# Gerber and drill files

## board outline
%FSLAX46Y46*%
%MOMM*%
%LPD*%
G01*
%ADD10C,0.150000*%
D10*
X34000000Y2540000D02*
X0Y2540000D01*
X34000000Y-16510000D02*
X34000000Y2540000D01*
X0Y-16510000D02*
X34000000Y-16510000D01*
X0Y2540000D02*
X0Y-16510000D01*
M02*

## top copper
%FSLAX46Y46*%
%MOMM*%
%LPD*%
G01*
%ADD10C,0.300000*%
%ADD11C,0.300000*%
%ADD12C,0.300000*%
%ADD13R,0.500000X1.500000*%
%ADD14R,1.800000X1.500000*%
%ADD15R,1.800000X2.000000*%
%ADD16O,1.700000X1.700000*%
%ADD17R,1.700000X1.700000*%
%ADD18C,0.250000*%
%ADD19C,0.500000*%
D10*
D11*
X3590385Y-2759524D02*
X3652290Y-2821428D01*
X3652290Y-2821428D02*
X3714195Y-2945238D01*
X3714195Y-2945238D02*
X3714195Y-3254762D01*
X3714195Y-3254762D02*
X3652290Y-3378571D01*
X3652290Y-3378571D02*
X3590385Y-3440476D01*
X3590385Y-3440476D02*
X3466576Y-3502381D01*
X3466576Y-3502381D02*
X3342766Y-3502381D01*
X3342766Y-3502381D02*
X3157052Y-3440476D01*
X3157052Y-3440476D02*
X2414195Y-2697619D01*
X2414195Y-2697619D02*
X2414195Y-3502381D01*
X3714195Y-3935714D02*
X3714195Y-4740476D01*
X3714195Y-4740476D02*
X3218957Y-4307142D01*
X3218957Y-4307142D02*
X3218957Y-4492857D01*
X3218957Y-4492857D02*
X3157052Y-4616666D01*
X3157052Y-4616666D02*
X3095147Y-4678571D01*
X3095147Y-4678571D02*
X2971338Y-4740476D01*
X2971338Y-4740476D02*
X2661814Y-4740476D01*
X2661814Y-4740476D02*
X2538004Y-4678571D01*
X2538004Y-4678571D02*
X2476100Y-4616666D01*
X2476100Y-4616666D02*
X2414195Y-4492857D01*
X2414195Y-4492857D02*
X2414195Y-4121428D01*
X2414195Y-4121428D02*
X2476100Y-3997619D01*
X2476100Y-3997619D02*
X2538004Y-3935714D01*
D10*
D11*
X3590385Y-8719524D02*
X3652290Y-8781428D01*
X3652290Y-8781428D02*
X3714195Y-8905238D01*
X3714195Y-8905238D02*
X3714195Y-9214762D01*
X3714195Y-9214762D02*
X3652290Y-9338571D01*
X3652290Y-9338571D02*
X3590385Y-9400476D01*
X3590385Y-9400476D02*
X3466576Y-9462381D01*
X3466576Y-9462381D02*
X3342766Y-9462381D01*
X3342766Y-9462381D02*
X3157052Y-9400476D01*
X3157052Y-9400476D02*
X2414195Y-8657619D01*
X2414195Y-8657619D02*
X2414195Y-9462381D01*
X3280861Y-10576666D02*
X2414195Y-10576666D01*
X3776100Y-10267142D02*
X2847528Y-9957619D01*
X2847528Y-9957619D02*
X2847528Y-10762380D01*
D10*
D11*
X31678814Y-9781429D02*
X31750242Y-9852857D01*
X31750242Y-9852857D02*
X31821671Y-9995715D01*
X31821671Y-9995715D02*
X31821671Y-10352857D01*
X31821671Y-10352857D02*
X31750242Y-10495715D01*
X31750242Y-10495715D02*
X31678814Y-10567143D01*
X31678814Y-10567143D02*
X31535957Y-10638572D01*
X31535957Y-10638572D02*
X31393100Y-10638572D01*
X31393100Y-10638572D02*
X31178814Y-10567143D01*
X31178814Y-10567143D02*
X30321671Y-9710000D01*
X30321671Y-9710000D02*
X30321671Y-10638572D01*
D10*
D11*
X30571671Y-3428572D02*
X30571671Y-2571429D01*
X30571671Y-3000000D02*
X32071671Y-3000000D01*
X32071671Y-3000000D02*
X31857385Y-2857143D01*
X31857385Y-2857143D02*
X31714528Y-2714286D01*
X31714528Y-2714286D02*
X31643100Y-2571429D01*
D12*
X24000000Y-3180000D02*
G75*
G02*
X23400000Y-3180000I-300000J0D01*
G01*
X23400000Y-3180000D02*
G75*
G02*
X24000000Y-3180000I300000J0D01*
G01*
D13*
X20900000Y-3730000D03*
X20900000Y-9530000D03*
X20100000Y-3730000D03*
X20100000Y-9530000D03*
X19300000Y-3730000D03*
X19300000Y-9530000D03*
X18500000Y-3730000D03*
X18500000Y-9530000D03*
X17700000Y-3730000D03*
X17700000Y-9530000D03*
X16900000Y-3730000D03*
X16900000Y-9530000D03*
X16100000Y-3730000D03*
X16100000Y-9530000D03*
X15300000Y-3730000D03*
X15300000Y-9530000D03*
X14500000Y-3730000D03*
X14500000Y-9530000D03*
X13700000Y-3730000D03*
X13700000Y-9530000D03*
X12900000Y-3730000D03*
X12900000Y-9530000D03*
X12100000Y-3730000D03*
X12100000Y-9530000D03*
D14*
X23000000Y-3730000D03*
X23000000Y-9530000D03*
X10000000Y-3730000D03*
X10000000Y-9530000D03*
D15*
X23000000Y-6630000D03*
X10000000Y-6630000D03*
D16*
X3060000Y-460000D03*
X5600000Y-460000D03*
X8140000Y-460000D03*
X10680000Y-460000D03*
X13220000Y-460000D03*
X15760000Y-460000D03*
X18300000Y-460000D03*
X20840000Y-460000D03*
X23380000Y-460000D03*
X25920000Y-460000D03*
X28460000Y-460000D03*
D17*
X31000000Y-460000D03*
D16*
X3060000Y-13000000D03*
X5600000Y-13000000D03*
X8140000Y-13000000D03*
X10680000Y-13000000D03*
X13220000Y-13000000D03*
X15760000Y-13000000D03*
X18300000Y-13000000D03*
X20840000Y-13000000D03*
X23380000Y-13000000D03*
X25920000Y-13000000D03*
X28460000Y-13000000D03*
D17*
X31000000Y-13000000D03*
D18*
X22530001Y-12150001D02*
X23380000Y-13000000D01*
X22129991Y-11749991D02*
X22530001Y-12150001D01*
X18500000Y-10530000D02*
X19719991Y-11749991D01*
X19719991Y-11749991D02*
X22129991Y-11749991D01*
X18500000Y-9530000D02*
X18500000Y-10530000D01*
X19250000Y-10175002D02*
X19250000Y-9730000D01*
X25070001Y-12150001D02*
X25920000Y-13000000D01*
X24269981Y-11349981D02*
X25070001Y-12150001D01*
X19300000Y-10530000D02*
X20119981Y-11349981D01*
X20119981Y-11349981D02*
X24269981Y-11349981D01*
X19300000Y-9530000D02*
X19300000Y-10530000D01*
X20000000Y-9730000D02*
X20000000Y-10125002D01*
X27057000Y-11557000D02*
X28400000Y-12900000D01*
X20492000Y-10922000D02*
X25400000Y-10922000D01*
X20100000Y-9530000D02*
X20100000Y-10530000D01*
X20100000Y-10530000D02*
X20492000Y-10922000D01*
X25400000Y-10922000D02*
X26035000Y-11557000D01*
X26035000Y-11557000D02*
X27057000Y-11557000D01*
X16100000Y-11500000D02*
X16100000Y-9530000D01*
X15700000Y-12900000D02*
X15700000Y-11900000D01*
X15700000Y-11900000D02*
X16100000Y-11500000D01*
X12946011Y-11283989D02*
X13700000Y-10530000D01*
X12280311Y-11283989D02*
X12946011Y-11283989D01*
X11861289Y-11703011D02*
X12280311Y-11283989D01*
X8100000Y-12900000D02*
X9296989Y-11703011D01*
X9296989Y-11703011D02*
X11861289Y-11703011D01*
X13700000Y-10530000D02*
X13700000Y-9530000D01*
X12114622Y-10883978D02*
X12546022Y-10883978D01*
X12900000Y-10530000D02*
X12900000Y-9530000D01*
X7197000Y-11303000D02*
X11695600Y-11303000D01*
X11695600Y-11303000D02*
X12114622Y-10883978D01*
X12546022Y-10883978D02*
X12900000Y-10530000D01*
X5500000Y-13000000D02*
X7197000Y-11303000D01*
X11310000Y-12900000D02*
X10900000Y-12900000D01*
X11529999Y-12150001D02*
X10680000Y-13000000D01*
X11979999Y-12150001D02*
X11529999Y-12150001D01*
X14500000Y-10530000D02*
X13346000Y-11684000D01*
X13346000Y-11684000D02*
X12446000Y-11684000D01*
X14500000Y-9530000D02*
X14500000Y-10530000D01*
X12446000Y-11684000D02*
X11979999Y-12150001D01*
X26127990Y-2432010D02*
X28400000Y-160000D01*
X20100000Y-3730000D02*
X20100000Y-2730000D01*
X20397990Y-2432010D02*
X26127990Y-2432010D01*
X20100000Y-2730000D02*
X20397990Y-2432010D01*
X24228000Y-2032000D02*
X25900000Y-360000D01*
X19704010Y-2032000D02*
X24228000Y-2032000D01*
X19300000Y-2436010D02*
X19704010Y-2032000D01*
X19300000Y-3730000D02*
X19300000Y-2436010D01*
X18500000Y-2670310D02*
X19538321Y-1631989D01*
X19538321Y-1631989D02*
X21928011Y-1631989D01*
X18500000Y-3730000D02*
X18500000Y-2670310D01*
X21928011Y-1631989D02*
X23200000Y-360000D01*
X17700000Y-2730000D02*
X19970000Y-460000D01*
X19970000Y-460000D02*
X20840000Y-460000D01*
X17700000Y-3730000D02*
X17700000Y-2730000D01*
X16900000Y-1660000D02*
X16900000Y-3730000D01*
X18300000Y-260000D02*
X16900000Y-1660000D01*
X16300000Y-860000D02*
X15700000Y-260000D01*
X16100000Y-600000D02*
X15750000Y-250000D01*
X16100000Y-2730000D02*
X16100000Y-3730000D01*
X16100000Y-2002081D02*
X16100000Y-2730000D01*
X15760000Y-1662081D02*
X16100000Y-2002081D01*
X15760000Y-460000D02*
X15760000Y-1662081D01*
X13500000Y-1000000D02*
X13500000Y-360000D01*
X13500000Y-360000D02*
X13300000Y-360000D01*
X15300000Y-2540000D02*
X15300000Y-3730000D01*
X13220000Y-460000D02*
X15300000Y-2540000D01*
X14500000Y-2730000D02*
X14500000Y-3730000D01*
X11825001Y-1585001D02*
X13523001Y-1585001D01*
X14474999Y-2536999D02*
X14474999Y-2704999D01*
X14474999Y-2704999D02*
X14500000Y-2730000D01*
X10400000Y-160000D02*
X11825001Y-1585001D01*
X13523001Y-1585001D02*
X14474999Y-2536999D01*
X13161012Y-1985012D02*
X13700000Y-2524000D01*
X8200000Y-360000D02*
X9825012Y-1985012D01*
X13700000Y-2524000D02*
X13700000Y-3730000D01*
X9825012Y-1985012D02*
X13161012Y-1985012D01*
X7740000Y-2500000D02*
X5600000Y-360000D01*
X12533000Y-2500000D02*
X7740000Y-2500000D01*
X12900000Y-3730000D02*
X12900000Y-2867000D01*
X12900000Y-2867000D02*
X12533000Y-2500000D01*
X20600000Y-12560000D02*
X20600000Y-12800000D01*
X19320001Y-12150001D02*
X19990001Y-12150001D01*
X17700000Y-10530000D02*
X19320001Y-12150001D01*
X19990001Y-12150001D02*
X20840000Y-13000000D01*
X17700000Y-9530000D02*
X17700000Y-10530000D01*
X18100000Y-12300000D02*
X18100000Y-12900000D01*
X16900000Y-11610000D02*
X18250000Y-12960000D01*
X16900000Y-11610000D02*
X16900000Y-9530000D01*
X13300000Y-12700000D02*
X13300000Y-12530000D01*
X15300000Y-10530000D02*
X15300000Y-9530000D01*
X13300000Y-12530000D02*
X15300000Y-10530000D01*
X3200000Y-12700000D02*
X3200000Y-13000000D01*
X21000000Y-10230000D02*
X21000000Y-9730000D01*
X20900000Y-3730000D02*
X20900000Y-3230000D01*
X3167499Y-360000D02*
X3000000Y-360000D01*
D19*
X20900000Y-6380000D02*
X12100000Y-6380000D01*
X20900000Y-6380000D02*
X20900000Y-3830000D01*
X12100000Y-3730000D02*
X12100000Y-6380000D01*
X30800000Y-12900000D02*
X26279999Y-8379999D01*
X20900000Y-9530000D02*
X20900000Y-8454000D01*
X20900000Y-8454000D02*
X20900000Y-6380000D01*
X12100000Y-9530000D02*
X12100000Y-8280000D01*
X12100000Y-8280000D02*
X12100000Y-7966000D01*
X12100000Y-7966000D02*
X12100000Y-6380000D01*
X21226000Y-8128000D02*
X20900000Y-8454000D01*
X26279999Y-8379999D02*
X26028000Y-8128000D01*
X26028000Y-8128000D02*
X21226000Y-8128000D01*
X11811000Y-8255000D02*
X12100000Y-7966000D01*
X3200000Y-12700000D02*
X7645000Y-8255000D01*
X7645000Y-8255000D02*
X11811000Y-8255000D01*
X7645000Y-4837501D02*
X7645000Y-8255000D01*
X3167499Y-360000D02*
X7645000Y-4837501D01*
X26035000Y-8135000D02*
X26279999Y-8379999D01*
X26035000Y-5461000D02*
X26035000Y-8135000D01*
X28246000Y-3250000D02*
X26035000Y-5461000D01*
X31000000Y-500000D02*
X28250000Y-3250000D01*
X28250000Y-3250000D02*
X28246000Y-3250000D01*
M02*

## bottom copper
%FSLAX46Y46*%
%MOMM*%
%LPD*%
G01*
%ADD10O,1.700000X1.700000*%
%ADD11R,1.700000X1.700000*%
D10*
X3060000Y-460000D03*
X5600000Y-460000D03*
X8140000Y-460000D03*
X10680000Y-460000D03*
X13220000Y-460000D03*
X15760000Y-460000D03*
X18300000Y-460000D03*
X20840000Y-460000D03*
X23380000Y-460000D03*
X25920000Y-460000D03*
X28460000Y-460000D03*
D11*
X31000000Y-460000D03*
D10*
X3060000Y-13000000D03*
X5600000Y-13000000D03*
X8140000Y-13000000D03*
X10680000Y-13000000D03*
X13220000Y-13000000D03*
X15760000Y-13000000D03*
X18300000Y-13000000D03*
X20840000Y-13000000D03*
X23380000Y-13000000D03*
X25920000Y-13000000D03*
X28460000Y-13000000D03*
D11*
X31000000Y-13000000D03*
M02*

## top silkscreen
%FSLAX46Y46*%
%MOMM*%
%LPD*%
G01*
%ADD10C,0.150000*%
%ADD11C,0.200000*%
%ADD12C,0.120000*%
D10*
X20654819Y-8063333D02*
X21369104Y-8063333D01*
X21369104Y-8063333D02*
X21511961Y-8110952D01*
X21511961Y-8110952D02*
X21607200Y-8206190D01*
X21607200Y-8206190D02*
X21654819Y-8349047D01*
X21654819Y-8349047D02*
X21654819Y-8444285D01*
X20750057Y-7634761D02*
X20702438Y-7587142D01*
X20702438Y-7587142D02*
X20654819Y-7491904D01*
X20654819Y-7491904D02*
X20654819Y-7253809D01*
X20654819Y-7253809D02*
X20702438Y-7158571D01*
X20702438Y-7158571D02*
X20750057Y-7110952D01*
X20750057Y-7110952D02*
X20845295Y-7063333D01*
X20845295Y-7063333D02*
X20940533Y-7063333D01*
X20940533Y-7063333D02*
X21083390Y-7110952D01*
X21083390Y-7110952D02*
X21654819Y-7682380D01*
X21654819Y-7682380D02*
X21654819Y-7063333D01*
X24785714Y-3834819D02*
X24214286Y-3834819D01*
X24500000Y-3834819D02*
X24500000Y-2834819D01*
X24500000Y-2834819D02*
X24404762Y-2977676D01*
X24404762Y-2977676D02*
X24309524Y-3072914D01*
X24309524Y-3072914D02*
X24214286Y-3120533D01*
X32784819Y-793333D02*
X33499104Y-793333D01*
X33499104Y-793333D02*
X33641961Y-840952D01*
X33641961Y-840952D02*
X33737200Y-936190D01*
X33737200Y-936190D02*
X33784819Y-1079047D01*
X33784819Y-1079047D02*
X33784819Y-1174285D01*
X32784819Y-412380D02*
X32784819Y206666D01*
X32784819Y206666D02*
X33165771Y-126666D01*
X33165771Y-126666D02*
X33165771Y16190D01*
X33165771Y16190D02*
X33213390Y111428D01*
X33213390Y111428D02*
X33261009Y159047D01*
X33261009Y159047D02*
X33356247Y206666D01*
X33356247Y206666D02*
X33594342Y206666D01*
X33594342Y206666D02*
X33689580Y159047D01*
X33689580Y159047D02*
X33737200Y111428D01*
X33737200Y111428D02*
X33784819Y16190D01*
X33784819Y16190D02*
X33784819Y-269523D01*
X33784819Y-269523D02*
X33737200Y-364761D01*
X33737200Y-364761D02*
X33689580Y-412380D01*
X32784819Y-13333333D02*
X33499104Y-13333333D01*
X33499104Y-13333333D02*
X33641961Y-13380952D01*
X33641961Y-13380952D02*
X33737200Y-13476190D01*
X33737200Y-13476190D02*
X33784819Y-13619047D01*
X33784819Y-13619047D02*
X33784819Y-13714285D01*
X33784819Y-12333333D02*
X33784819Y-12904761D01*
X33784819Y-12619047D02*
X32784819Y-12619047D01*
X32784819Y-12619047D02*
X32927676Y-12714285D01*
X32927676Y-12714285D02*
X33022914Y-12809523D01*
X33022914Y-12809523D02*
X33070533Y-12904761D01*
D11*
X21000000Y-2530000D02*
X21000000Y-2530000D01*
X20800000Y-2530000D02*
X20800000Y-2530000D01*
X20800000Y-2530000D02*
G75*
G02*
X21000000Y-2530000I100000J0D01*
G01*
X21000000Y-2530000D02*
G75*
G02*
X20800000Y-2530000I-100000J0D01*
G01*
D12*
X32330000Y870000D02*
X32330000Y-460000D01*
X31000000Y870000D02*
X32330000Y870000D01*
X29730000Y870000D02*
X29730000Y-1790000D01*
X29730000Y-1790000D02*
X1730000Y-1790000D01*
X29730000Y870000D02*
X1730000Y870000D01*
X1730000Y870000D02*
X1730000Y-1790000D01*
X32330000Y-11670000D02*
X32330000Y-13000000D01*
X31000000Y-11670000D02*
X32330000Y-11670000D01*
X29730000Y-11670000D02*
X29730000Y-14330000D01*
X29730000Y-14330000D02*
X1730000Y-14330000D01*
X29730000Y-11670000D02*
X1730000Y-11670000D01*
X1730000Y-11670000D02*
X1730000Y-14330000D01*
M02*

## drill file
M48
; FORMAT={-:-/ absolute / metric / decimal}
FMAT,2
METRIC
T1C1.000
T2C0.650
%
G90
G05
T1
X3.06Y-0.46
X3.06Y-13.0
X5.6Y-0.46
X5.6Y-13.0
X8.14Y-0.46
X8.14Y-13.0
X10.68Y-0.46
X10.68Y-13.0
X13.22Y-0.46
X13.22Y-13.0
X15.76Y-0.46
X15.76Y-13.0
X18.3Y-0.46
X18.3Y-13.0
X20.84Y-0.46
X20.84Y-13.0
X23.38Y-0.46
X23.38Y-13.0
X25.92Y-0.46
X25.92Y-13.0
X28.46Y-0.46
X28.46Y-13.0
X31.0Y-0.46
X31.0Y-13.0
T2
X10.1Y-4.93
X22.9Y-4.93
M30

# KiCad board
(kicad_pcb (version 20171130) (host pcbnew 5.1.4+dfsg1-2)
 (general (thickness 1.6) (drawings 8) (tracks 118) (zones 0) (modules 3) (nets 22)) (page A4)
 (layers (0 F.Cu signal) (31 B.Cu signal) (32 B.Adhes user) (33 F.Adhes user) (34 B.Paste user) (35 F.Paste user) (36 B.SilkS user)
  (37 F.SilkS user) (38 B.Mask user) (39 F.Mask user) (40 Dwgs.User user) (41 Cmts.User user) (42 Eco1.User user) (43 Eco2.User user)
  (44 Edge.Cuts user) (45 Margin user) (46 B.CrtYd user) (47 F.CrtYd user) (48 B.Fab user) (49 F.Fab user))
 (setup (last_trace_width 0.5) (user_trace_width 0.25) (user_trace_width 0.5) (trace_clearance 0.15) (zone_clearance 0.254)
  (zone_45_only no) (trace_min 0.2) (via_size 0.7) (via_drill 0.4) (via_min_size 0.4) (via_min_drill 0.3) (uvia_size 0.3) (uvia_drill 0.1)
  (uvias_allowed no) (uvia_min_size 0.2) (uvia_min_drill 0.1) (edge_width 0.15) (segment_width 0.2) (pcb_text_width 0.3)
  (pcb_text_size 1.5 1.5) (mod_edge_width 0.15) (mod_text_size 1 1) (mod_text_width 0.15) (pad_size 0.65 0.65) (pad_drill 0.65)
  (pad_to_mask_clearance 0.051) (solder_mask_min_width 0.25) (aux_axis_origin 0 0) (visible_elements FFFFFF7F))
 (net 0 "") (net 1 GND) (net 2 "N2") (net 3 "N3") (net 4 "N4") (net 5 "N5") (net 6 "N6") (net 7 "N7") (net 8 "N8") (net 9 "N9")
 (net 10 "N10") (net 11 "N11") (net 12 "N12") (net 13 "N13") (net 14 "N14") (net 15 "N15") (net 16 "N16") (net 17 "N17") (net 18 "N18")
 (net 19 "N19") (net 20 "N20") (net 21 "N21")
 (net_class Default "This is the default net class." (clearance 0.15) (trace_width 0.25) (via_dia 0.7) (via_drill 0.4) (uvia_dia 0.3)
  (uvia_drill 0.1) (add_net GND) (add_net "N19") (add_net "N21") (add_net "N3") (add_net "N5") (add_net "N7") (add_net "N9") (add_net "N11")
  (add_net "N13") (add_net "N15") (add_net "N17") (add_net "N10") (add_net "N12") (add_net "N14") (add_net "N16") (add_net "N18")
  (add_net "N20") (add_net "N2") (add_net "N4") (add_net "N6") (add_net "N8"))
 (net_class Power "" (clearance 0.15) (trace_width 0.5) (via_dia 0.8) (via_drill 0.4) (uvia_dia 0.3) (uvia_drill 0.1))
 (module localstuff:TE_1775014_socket (layer F.Cu) (at 16.5 6.63 180)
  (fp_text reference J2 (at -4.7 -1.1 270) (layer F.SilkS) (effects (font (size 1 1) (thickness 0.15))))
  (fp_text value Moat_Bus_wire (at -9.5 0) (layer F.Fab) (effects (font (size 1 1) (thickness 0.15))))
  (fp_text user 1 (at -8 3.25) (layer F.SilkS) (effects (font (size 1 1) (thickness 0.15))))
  (fp_circle (center -7.2 3.45) (end -6.9 3.45) (layer F.Cu) (width 0.3))
  (fp_line (start -4.5 4.1) (end -4.5 4.1) (layer F.SilkS) (width 0.2))
  (fp_line (start -4.3 4.1) (end -4.3 4.1) (layer F.SilkS) (width 0.2))
  (fp_arc (start -4.4 4.1) (end -4.5 4.1) (angle -180) (layer F.SilkS) (width 0.2))
  (fp_arc (start -4.4 4.1) (end -4.3 4.1) (angle -180) (layer F.SilkS) (width 0.2))
  (pad 1 smd rect (at -4.4 2.9 180) (size 0.5 1.5) (layers F.Cu F.Paste) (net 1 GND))
  (pad 2 smd rect (at -4.4 -2.9 180) (size 0.5 1.5) (layers F.Cu F.Paste) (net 1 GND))
  (pad 3 smd rect (at -3.6 2.9 180) (size 0.5 1.5) (layers F.Cu F.Paste) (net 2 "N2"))
  (pad 4 smd rect (at -3.6 -2.9 180) (size 0.5 1.5) (layers F.Cu F.Paste) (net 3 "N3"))
  (pad 5 smd rect (at -2.8 2.9 180) (size 0.5 1.5) (layers F.Cu F.Paste) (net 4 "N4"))
  (pad 6 smd rect (at -2.8 -2.9 180) (size 0.5 1.5) (layers F.Cu F.Paste) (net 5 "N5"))
  (pad 7 smd rect (at -2 2.9 180) (size 0.5 1.5) (layers F.Cu F.Paste) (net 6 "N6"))
  (pad 8 smd rect (at -2 -2.9 180) (size 0.5 1.5) (layers F.Cu F.Paste) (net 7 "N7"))
  (pad 9 smd rect (at -1.2 2.9 180) (size 0.5 1.5) (layers F.Cu F.Paste) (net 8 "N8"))
  (pad 10 smd rect (at -1.2 -2.9 180) (size 0.5 1.5) (layers F.Cu F.Paste) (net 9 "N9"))
  (pad 11 smd rect (at -0.4 2.9 180) (size 0.5 1.5) (layers F.Cu F.Paste) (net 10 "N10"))
  (pad 12 smd rect (at -0.4 -2.9 180) (size 0.5 1.5) (layers F.Cu F.Paste) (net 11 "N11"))
  (pad 13 smd rect (at 0.4 2.9 180) (size 0.5 1.5) (layers F.Cu F.Paste) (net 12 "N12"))
  (pad 14 smd rect (at 0.4 -2.9 180) (size 0.5 1.5) (layers F.Cu F.Paste) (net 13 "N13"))
  (pad 15 smd rect (at 1.2 2.9 180) (size 0.5 1.5) (layers F.Cu F.Paste) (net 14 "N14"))
  (pad 16 smd rect (at 1.2 -2.9 180) (size 0.5 1.5) (layers F.Cu F.Paste) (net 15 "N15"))
  (pad 17 smd rect (at 2 2.9 180) (size 0.5 1.5) (layers F.Cu F.Paste) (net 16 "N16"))
  (pad 18 smd rect (at 2 -2.9 180) (size 0.5 1.5) (layers F.Cu F.Paste) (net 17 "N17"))
  (pad 19 smd rect (at 2.8 2.9 180) (size 0.5 1.5) (layers F.Cu F.Paste) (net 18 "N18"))
  (pad 20 smd rect (at 2.8 -2.9 180) (size 0.5 1.5) (layers F.Cu F.Paste) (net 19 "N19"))
  (pad 21 smd rect (at 3.6 2.9 180) (size 0.5 1.5) (layers F.Cu F.Paste) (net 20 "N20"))
  (pad 22 smd rect (at 3.6 -2.9 180) (size 0.5 1.5) (layers F.Cu F.Paste) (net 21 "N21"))
  (pad 23 smd rect (at 4.4 2.9 180) (size 0.5 1.5) (layers F.Cu F.Paste) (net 1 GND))
  (pad 24 smd rect (at 4.4 -2.9 180) (size 0.5 1.5) (layers F.Cu F.Paste) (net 1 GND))
  (pad MNT smd rect (at -6.5 2.9 270) (size 1.5 1.8) (layers F.Cu F.Paste))
  (pad MNT smd rect (at -6.5 -2.9 270) (size 1.5 1.8) (layers F.Cu F.Paste))
  (pad MNT smd rect (at 6.5 2.9 270) (size 1.5 1.8) (layers F.Cu F.Paste))
  (pad MNT smd rect (at 6.5 -2.9 270) (size 1.5 1.8) (layers F.Cu F.Paste))
  (pad MNT smd rect (at -6.5 0 180) (size 1.8 2) (layers F.Cu F.Paste))
  (pad MNT smd rect (at 6.5 0 180) (size 1.8 2) (layers F.Cu F.Paste))
  (pad "" np_thru_hole circle (at -6.4 1.7 180) (size 0.65 0.65) (drill 0.65) (layers *.Cu *.Mask))
  (pad "" np_thru_hole circle (at 6.4 1.7 180) (size 0.65 0.65) (drill 0.65) (layers *.Cu *.Mask)))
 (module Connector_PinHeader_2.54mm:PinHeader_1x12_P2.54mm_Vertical (layer F.Cu) (at 31 0.46 270)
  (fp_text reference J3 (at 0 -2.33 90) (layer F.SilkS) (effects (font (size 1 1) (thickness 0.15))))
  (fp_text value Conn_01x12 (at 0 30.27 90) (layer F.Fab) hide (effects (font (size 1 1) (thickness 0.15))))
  (fp_line (start -1.33 -1.33) (end 0 -1.33) (layer F.SilkS) (width 0.12))
  (fp_line (start -1.33 0) (end -1.33 -1.33) (layer F.SilkS) (width 0.12))
  (fp_line (start -1.33 1.27) (end 1.33 1.27) (layer F.SilkS) (width 0.12))
  (fp_line (start 1.33 1.27) (end 1.33 29.27) (layer F.SilkS) (width 0.12))
  (fp_line (start -1.33 1.27) (end -1.33 29.27) (layer F.SilkS) (width 0.12))
  (fp_line (start -1.33 29.27) (end 1.33 29.27) (layer F.SilkS) (width 0.12))
  (pad 12 thru_hole oval (at 0 27.94 270) (size 1.7 1.7) (drill 1) (layers *.Cu *.Mask) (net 1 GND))
  (pad 11 thru_hole oval (at 0 25.4 270) (size 1.7 1.7) (drill 1) (layers *.Cu *.Mask) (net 20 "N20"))
  (pad 10 thru_hole oval (at 0 22.86 270) (size 1.7 1.7) (drill 1) (layers *.Cu *.Mask) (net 18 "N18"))
  (pad 9 thru_hole oval (at 0 20.32 270) (size 1.7 1.7) (drill 1) (layers *.Cu *.Mask) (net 16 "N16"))
  (pad 8 thru_hole oval (at 0 17.78 270) (size 1.7 1.7) (drill 1) (layers *.Cu *.Mask) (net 14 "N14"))
  (pad 7 thru_hole oval (at 0 15.24 270) (size 1.7 1.7) (drill 1) (layers *.Cu *.Mask) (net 12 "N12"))
  (pad 6 thru_hole oval (at 0 12.7 270) (size 1.7 1.7) (drill 1) (layers *.Cu *.Mask) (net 10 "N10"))
  (pad 5 thru_hole oval (at 0 10.16 270) (size 1.7 1.7) (drill 1) (layers *.Cu *.Mask) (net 8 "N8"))
  (pad 4 thru_hole oval (at 0 7.62 270) (size 1.7 1.7) (drill 1) (layers *.Cu *.Mask) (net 6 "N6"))
  (pad 3 thru_hole oval (at 0 5.08 270) (size 1.7 1.7) (drill 1) (layers *.Cu *.Mask) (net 4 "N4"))
  (pad 2 thru_hole oval (at 0 2.54 270) (size 1.7 1.7) (drill 1) (layers *.Cu *.Mask) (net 2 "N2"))
  (pad 1 thru_hole rect (at 0 0 270) (size 1.7 1.7) (drill 1) (layers *.Cu *.Mask) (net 1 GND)))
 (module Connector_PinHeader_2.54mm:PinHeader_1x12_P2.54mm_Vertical (layer F.Cu) (at 31 13 270)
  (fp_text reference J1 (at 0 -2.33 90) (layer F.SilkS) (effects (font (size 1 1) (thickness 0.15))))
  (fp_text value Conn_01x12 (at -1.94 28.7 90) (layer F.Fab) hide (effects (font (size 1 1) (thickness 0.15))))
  (fp_line (start -1.33 -1.33) (end 0 -1.33) (layer F.SilkS) (width 0.12))
  (fp_line (start -1.33 0) (end -1.33 -1.33) (layer F.SilkS) (width 0.12))
  (fp_line (start -1.33 1.27) (end 1.33 1.27) (layer F.SilkS) (width 0.12))
  (fp_line (start 1.33 1.27) (end 1.33 29.27) (layer F.SilkS) (width 0.12))
  (fp_line (start -1.33 1.27) (end -1.33 29.27) (layer F.SilkS) (width 0.12))
  (fp_line (start -1.33 29.27) (end 1.33 29.27) (layer F.SilkS) (width 0.12))
  (pad 12 thru_hole oval (at 0 27.94 270) (size 1.7 1.7) (drill 1) (layers *.Cu *.Mask) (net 1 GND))
  (pad 11 thru_hole oval (at 0 25.4 270) (size 1.7 1.7) (drill 1) (layers *.Cu *.Mask) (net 21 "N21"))
  (pad 10 thru_hole oval (at 0 22.86 270) (size 1.7 1.7) (drill 1) (layers *.Cu *.Mask) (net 19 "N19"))
  (pad 9 thru_hole oval (at 0 20.32 270) (size 1.7 1.7) (drill 1) (layers *.Cu *.Mask) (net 17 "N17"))
  (pad 8 thru_hole oval (at 0 17.78 270) (size 1.7 1.7) (drill 1) (layers *.Cu *.Mask) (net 15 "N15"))
  (pad 7 thru_hole oval (at 0 15.24 270) (size 1.7 1.7) (drill 1) (layers *.Cu *.Mask) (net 13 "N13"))
  (pad 6 thru_hole oval (at 0 12.7 270) (size 1.7 1.7) (drill 1) (layers *.Cu *.Mask) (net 11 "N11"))
  (pad 5 thru_hole oval (at 0 10.16 270) (size 1.7 1.7) (drill 1) (layers *.Cu *.Mask) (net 9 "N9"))
  (pad 4 thru_hole oval (at 0 7.62 270) (size 1.7 1.7) (drill 1) (layers *.Cu *.Mask) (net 7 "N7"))
  (pad 3 thru_hole oval (at 0 5.08 270) (size 1.7 1.7) (drill 1) (layers *.Cu *.Mask) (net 5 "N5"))
  (pad 2 thru_hole oval (at 0 2.54 270) (size 1.7 1.7) (drill 1) (layers *.Cu *.Mask) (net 3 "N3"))
  (pad 1 thru_hole rect (at 0 0 270) (size 1.7 1.7) (drill 1) (layers *.Cu *.Mask) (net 1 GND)))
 (gr_line (start 34 -2.54) (end 0 -2.54) (layer Edge.Cuts) (width 0.15))
 (gr_line (start 34 16.51) (end 34 -2.54) (layer Edge.Cuts) (width 0.15))
 (gr_line (start 0 16.51) (end 34 16.51) (layer Edge.Cuts) (width 0.15))
 (gr_line (start 0 -2.54) (end 0 16.51) (layer Edge.Cuts) (width 0.15))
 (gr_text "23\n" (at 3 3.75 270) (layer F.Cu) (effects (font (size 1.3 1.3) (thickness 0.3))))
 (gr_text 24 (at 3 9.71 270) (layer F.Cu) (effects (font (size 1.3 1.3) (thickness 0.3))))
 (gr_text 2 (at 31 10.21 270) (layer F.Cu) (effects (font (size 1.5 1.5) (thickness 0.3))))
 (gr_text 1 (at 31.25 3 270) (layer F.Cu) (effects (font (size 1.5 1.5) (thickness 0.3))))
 (segment (start 22.530001 12.150001) (end 23.38 13) (width 0.25) (layer F.Cu) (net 7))
 (segment (start 22.129991 11.749991) (end 22.530001 12.150001) (width 0.25) (layer F.Cu) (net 7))
 (segment (start 18.5 10.53) (end 19.719991 11.749991) (width 0.25) (layer F.Cu) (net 7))
 (segment (start 19.719991 11.749991) (end 22.129991 11.749991) (width 0.25) (layer F.Cu) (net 7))
 (segment (start 18.5 9.53) (end 18.5 10.53) (width 0.25) (layer F.Cu) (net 7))
 (segment (start 19.25 10.175002) (end 19.25 9.73) (width 0.25) (layer F.Cu) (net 5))
 (segment (start 25.070001 12.150001) (end 25.92 13) (width 0.25) (layer F.Cu) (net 5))
 (segment (start 24.269981 11.349981) (end 25.070001 12.150001) (width 0.25) (layer F.Cu) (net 5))
 (segment (start 19.3 10.53) (end 20.119981 11.349981) (width 0.25) (layer F.Cu) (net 5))
 (segment (start 20.119981 11.349981) (end 24.269981 11.349981) (width 0.25) (layer F.Cu) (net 5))
 (segment (start 19.3 9.53) (end 19.3 10.53) (width 0.25) (layer F.Cu) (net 5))
 (segment (start 20 9.73) (end 20 10.125002) (width 0.25) (layer F.Cu) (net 3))
 (segment (start 27.057 11.557) (end 28.4 12.9) (width 0.25) (layer F.Cu) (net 3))
 (segment (start 20.492 10.922) (end 25.4 10.922) (width 0.25) (layer F.Cu) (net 3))
 (segment (start 20.1 9.53) (end 20.1 10.53) (width 0.25) (layer F.Cu) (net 3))
 (segment (start 20.1 10.53) (end 20.492 10.922) (width 0.25) (layer F.Cu) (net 3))
 (segment (start 25.4 10.922) (end 26.035 11.557) (width 0.25) (layer F.Cu) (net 3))
 (segment (start 26.035 11.557) (end 27.057 11.557) (width 0.25) (layer F.Cu) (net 3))
 (segment (start 16.1 11.5) (end 16.1 9.53) (width 0.25) (layer F.Cu) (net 13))
 (segment (start 15.7 12.9) (end 15.7 11.9) (width 0.25) (layer F.Cu) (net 13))
 (segment (start 15.7 11.9) (end 16.1 11.5) (width 0.25) (layer F.Cu) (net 13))
 (segment (start 12.946011 11.283989) (end 13.7 10.53) (width 0.25) (layer F.Cu) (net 19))
 (segment (start 12.280311 11.283989) (end 12.946011 11.283989) (width 0.25) (layer F.Cu) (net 19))
 (segment (start 11.861289 11.703011) (end 12.280311 11.283989) (width 0.25) (layer F.Cu) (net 19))
 (segment (start 8.1 12.9) (end 9.296989 11.703011) (width 0.25) (layer F.Cu) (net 19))
 (segment (start 9.296989 11.703011) (end 11.861289 11.703011) (width 0.25) (layer F.Cu) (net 19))
 (segment (start 13.7 10.53) (end 13.7 9.53) (width 0.25) (layer F.Cu) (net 19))
 (segment (start 12.114622 10.883978) (end 12.546022 10.883978) (width 0.25) (layer F.Cu) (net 21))
 (segment (start 12.9 10.53) (end 12.9 9.53) (width 0.25) (layer F.Cu) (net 21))
 (segment (start 7.197 11.303) (end 11.6956 11.303) (width 0.25) (layer F.Cu) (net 21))
 (segment (start 11.6956 11.303) (end 12.114622 10.883978) (width 0.25) (layer F.Cu) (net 21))
 (segment (start 12.546022 10.883978) (end 12.9 10.53) (width 0.25) (layer F.Cu) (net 21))
 (segment (start 5.5 13) (end 7.197 11.303) (width 0.25) (layer F.Cu) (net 21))
 (segment (start 11.31 12.9) (end 10.9 12.9) (width 0.25) (layer F.Cu) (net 17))
 (segment (start 11.529999 12.150001) (end 10.68 13) (width 0.25) (layer F.Cu) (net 17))
 (segment (start 11.979999 12.150001) (end 11.529999 12.150001) (width 0.25) (layer F.Cu) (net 17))
 (segment (start 14.5 10.53) (end 13.346 11.684) (width 0.25) (layer F.Cu) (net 17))
 (segment (start 13.346 11.684) (end 12.446 11.684) (width 0.25) (layer F.Cu) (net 17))
 (segment (start 14.5 9.53) (end 14.5 10.53) (width 0.25) (layer F.Cu) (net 17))
 (segment (start 12.446 11.684) (end 11.979999 12.150001) (width 0.25) (layer F.Cu) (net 17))
 (segment (start 26.12799 2.43201) (end 28.4 0.16) (width 0.25) (layer F.Cu) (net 2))
 (segment (start 20.1 3.73) (end 20.1 2.73) (width 0.25) (layer F.Cu) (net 2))
 (segment (start 20.39799 2.43201) (end 26.12799 2.43201) (width 0.25) (layer F.Cu) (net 2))
 (segment (start 20.1 2.73) (end 20.39799 2.43201) (width 0.25) (layer F.Cu) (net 2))
 (segment (start 24.228 2.032) (end 25.9 0.36) (width 0.25) (layer F.Cu) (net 4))
 (segment (start 19.70401 2.032) (end 24.228 2.032) (width 0.25) (layer F.Cu) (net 4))
 (segment (start 19.3 2.43601) (end 19.70401 2.032) (width 0.25) (layer F.Cu) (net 4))
 (segment (start 19.3 3.73) (end 19.3 2.43601) (width 0.25) (layer F.Cu) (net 4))
 (segment (start 18.5 2.67031) (end 19.538321 1.631989) (width 0.25) (layer F.Cu) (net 6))
 (segment (start 19.538321 1.631989) (end 21.928011 1.631989) (width 0.25) (layer F.Cu) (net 6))
 (segment (start 18.5 3.73) (end 18.5 2.67031) (width 0.25) (layer F.Cu) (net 6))
 (segment (start 21.928011 1.631989) (end 23.2 0.36) (width 0.25) (layer F.Cu) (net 6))
 (segment (start 17.7 2.73) (end 19.97 0.46) (width 0.25) (layer F.Cu) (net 8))
 (segment (start 19.97 0.46) (end 20.84 0.46) (width 0.25) (layer F.Cu) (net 8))
 (segment (start 17.7 3.73) (end 17.7 2.73) (width 0.25) (layer F.Cu) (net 8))
 (segment (start 16.9 1.66) (end 16.9 3.73) (width 0.25) (layer F.Cu) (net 10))
 (segment (start 18.3 0.26) (end 16.9 1.66) (width 0.25) (layer F.Cu) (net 10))
 (segment (start 16.3 0.86) (end 15.7 0.26) (width 0.25) (layer F.Cu) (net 12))
 (segment (start 16.1 0.6) (end 15.75 0.25) (width 0.25) (layer F.Cu) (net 12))
 (segment (start 16.1 2.73) (end 16.1 3.73) (width 0.25) (layer F.Cu) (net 12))
 (segment (start 16.1 2.002081) (end 16.1 2.73) (width 0.25) (layer F.Cu) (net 12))
 (segment (start 15.76 1.662081) (end 16.1 2.002081) (width 0.25) (layer F.Cu) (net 12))
 (segment (start 15.76 0.46) (end 15.76 1.662081) (width 0.25) (layer F.Cu) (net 12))
 (segment (start 13.5 1) (end 13.5 0.36) (width 0.25) (layer F.Cu) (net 14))
 (segment (start 13.5 0.36) (end 13.3 0.36) (width 0.25) (layer F.Cu) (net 14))
 (segment (start 15.3 2.54) (end 15.3 3.73) (width 0.25) (layer F.Cu) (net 14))
 (segment (start 13.22 0.46) (end 15.3 2.54) (width 0.25) (layer F.Cu) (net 14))
 (segment (start 14.5 2.73) (end 14.5 3.73) (width 0.25) (layer F.Cu) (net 16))
 (segment (start 11.825001 1.585001) (end 13.523001 1.585001) (width 0.25) (layer F.Cu) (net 16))
 (segment (start 14.474999 2.536999) (end 14.474999 2.704999) (width 0.25) (layer F.Cu) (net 16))
 (segment (start 14.474999 2.704999) (end 14.5 2.73) (width 0.25) (layer F.Cu) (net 16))
 (segment (start 10.4 0.16) (end 11.825001 1.585001) (width 0.25) (layer F.Cu) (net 16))
 (segment (start 13.523001 1.585001) (end 14.474999 2.536999) (width 0.25) (layer F.Cu) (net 16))
 (segment (start 13.161012 1.985012) (end 13.7 2.524) (width 0.25) (layer F.Cu) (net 18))
 (segment (start 8.2 0.36) (end 9.825012 1.985012) (width 0.25) (layer F.Cu) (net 18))
 (segment (start 13.7 2.524) (end 13.7 3.73) (width 0.25) (layer F.Cu) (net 18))
 (segment (start 9.825012 1.985012) (end 13.161012 1.985012) (width 0.25) (layer F.Cu) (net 18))
 (segment (start 7.74 2.5) (end 5.6 0.36) (width 0.25) (layer F.Cu) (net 20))
 (segment (start 12.533 2.5) (end 7.74 2.5) (width 0.25) (layer F.Cu) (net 20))
 (segment (start 12.9 3.73) (end 12.9 2.867) (width 0.25) (layer F.Cu) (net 20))
 (segment (start 12.9 2.867) (end 12.533 2.5) (width 0.25) (layer F.Cu) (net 20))
 (segment (start 20.6 12.56) (end 20.6 12.8) (width 0.25) (layer F.Cu) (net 9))
 (segment (start 19.320001 12.150001) (end 19.990001 12.150001) (width 0.25) (layer F.Cu) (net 9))
 (segment (start 17.7 10.53) (end 19.320001 12.150001) (width 0.25) (layer F.Cu) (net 9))
 (segment (start 19.990001 12.150001) (end 20.84 13) (width 0.25) (layer F.Cu) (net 9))
 (segment (start 17.7 9.53) (end 17.7 10.53) (width 0.25) (layer F.Cu) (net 9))
 (segment (start 18.1 12.3) (end 18.1 12.9) (width 0.25) (layer F.Cu) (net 11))
 (segment (start 16.9 11.61) (end 18.25 12.96) (width 0.25) (layer F.Cu) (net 11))
 (segment (start 16.9 11.61) (end 16.9 9.53) (width 0.25) (layer F.Cu) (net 11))
 (segment (start 13.3 12.7) (end 13.3 12.53) (width 0.25) (layer F.Cu) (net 15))
 (segment (start 15.3 10.53) (end 15.3 9.53) (width 0.25) (layer F.Cu) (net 15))
 (segment (start 13.3 12.53) (end 15.3 10.53) (width 0.25) (layer F.Cu) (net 15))
 (segment (start 3.2 12.7) (end 3.2 13) (width 0.25) (layer F.Cu) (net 1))
 (segment (start 21 10.23) (end 21 9.73) (width 0.25) (layer F.Cu) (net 1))
 (segment (start 20.9 3.73) (end 20.9 3.23) (width 0.25) (layer F.Cu) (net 1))
 (segment (start 3.167499 0.36) (end 3 0.36) (width 0.25) (layer F.Cu) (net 1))
 (segment (start 20.9 6.38) (end 12.1 6.38) (width 0.5) (layer F.Cu) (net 1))
 (segment (start 20.9 6.38) (end 20.9 3.83) (width 0.5) (layer F.Cu) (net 1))
 (segment (start 12.1 3.73) (end 12.1 6.38) (width 0.5) (layer F.Cu) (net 1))
 (segment (start 30.8 12.9) (end 26.279999 8.379999) (width 0.5) (layer F.Cu) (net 1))
 (segment (start 20.9 9.53) (end 20.9 8.454) (width 0.5) (layer F.Cu) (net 1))
 (segment (start 20.9 8.454) (end 20.9 6.38) (width 0.5) (layer F.Cu) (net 1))
 (segment (start 12.1 9.53) (end 12.1 8.28) (width 0.5) (layer F.Cu) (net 1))
 (segment (start 12.1 8.28) (end 12.1 7.966) (width 0.5) (layer F.Cu) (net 1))
 (segment (start 12.1 7.966) (end 12.1 6.38) (width 0.5) (layer F.Cu) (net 1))
 (segment (start 21.226 8.128) (end 20.9 8.454) (width 0.5) (layer F.Cu) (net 1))
 (segment (start 26.279999 8.379999) (end 26.028 8.128) (width 0.5) (layer F.Cu) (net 1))
 (segment (start 26.028 8.128) (end 21.226 8.128) (width 0.5) (layer F.Cu) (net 1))
 (segment (start 11.811 8.255) (end 12.1 7.966) (width 0.5) (layer F.Cu) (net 1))
 (segment (start 3.2 12.7) (end 7.645 8.255) (width 0.5) (layer F.Cu) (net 1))
 (segment (start 7.645 8.255) (end 11.811 8.255) (width 0.5) (layer F.Cu) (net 1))
 (segment (start 7.645 4.837501) (end 7.645 8.255) (width 0.5) (layer F.Cu) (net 1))
 (segment (start 3.167499 0.36) (end 7.645 4.837501) (width 0.5) (layer F.Cu) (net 1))
 (segment (start 26.035 8.135) (end 26.279999 8.379999) (width 0.5) (layer F.Cu) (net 1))
 (segment (start 26.035 5.461) (end 26.035 8.135) (width 0.5) (layer F.Cu) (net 1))
 (segment (start 28.246 3.25) (end 26.035 5.461) (width 0.5) (layer F.Cu) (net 1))
 (segment (start 31 0.5) (end 28.25 3.25) (width 0.5) (layer F.Cu) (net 1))
 (segment (start 28.25 3.25) (end 28.246 3.25) (width 0.5) (layer F.Cu) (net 1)))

